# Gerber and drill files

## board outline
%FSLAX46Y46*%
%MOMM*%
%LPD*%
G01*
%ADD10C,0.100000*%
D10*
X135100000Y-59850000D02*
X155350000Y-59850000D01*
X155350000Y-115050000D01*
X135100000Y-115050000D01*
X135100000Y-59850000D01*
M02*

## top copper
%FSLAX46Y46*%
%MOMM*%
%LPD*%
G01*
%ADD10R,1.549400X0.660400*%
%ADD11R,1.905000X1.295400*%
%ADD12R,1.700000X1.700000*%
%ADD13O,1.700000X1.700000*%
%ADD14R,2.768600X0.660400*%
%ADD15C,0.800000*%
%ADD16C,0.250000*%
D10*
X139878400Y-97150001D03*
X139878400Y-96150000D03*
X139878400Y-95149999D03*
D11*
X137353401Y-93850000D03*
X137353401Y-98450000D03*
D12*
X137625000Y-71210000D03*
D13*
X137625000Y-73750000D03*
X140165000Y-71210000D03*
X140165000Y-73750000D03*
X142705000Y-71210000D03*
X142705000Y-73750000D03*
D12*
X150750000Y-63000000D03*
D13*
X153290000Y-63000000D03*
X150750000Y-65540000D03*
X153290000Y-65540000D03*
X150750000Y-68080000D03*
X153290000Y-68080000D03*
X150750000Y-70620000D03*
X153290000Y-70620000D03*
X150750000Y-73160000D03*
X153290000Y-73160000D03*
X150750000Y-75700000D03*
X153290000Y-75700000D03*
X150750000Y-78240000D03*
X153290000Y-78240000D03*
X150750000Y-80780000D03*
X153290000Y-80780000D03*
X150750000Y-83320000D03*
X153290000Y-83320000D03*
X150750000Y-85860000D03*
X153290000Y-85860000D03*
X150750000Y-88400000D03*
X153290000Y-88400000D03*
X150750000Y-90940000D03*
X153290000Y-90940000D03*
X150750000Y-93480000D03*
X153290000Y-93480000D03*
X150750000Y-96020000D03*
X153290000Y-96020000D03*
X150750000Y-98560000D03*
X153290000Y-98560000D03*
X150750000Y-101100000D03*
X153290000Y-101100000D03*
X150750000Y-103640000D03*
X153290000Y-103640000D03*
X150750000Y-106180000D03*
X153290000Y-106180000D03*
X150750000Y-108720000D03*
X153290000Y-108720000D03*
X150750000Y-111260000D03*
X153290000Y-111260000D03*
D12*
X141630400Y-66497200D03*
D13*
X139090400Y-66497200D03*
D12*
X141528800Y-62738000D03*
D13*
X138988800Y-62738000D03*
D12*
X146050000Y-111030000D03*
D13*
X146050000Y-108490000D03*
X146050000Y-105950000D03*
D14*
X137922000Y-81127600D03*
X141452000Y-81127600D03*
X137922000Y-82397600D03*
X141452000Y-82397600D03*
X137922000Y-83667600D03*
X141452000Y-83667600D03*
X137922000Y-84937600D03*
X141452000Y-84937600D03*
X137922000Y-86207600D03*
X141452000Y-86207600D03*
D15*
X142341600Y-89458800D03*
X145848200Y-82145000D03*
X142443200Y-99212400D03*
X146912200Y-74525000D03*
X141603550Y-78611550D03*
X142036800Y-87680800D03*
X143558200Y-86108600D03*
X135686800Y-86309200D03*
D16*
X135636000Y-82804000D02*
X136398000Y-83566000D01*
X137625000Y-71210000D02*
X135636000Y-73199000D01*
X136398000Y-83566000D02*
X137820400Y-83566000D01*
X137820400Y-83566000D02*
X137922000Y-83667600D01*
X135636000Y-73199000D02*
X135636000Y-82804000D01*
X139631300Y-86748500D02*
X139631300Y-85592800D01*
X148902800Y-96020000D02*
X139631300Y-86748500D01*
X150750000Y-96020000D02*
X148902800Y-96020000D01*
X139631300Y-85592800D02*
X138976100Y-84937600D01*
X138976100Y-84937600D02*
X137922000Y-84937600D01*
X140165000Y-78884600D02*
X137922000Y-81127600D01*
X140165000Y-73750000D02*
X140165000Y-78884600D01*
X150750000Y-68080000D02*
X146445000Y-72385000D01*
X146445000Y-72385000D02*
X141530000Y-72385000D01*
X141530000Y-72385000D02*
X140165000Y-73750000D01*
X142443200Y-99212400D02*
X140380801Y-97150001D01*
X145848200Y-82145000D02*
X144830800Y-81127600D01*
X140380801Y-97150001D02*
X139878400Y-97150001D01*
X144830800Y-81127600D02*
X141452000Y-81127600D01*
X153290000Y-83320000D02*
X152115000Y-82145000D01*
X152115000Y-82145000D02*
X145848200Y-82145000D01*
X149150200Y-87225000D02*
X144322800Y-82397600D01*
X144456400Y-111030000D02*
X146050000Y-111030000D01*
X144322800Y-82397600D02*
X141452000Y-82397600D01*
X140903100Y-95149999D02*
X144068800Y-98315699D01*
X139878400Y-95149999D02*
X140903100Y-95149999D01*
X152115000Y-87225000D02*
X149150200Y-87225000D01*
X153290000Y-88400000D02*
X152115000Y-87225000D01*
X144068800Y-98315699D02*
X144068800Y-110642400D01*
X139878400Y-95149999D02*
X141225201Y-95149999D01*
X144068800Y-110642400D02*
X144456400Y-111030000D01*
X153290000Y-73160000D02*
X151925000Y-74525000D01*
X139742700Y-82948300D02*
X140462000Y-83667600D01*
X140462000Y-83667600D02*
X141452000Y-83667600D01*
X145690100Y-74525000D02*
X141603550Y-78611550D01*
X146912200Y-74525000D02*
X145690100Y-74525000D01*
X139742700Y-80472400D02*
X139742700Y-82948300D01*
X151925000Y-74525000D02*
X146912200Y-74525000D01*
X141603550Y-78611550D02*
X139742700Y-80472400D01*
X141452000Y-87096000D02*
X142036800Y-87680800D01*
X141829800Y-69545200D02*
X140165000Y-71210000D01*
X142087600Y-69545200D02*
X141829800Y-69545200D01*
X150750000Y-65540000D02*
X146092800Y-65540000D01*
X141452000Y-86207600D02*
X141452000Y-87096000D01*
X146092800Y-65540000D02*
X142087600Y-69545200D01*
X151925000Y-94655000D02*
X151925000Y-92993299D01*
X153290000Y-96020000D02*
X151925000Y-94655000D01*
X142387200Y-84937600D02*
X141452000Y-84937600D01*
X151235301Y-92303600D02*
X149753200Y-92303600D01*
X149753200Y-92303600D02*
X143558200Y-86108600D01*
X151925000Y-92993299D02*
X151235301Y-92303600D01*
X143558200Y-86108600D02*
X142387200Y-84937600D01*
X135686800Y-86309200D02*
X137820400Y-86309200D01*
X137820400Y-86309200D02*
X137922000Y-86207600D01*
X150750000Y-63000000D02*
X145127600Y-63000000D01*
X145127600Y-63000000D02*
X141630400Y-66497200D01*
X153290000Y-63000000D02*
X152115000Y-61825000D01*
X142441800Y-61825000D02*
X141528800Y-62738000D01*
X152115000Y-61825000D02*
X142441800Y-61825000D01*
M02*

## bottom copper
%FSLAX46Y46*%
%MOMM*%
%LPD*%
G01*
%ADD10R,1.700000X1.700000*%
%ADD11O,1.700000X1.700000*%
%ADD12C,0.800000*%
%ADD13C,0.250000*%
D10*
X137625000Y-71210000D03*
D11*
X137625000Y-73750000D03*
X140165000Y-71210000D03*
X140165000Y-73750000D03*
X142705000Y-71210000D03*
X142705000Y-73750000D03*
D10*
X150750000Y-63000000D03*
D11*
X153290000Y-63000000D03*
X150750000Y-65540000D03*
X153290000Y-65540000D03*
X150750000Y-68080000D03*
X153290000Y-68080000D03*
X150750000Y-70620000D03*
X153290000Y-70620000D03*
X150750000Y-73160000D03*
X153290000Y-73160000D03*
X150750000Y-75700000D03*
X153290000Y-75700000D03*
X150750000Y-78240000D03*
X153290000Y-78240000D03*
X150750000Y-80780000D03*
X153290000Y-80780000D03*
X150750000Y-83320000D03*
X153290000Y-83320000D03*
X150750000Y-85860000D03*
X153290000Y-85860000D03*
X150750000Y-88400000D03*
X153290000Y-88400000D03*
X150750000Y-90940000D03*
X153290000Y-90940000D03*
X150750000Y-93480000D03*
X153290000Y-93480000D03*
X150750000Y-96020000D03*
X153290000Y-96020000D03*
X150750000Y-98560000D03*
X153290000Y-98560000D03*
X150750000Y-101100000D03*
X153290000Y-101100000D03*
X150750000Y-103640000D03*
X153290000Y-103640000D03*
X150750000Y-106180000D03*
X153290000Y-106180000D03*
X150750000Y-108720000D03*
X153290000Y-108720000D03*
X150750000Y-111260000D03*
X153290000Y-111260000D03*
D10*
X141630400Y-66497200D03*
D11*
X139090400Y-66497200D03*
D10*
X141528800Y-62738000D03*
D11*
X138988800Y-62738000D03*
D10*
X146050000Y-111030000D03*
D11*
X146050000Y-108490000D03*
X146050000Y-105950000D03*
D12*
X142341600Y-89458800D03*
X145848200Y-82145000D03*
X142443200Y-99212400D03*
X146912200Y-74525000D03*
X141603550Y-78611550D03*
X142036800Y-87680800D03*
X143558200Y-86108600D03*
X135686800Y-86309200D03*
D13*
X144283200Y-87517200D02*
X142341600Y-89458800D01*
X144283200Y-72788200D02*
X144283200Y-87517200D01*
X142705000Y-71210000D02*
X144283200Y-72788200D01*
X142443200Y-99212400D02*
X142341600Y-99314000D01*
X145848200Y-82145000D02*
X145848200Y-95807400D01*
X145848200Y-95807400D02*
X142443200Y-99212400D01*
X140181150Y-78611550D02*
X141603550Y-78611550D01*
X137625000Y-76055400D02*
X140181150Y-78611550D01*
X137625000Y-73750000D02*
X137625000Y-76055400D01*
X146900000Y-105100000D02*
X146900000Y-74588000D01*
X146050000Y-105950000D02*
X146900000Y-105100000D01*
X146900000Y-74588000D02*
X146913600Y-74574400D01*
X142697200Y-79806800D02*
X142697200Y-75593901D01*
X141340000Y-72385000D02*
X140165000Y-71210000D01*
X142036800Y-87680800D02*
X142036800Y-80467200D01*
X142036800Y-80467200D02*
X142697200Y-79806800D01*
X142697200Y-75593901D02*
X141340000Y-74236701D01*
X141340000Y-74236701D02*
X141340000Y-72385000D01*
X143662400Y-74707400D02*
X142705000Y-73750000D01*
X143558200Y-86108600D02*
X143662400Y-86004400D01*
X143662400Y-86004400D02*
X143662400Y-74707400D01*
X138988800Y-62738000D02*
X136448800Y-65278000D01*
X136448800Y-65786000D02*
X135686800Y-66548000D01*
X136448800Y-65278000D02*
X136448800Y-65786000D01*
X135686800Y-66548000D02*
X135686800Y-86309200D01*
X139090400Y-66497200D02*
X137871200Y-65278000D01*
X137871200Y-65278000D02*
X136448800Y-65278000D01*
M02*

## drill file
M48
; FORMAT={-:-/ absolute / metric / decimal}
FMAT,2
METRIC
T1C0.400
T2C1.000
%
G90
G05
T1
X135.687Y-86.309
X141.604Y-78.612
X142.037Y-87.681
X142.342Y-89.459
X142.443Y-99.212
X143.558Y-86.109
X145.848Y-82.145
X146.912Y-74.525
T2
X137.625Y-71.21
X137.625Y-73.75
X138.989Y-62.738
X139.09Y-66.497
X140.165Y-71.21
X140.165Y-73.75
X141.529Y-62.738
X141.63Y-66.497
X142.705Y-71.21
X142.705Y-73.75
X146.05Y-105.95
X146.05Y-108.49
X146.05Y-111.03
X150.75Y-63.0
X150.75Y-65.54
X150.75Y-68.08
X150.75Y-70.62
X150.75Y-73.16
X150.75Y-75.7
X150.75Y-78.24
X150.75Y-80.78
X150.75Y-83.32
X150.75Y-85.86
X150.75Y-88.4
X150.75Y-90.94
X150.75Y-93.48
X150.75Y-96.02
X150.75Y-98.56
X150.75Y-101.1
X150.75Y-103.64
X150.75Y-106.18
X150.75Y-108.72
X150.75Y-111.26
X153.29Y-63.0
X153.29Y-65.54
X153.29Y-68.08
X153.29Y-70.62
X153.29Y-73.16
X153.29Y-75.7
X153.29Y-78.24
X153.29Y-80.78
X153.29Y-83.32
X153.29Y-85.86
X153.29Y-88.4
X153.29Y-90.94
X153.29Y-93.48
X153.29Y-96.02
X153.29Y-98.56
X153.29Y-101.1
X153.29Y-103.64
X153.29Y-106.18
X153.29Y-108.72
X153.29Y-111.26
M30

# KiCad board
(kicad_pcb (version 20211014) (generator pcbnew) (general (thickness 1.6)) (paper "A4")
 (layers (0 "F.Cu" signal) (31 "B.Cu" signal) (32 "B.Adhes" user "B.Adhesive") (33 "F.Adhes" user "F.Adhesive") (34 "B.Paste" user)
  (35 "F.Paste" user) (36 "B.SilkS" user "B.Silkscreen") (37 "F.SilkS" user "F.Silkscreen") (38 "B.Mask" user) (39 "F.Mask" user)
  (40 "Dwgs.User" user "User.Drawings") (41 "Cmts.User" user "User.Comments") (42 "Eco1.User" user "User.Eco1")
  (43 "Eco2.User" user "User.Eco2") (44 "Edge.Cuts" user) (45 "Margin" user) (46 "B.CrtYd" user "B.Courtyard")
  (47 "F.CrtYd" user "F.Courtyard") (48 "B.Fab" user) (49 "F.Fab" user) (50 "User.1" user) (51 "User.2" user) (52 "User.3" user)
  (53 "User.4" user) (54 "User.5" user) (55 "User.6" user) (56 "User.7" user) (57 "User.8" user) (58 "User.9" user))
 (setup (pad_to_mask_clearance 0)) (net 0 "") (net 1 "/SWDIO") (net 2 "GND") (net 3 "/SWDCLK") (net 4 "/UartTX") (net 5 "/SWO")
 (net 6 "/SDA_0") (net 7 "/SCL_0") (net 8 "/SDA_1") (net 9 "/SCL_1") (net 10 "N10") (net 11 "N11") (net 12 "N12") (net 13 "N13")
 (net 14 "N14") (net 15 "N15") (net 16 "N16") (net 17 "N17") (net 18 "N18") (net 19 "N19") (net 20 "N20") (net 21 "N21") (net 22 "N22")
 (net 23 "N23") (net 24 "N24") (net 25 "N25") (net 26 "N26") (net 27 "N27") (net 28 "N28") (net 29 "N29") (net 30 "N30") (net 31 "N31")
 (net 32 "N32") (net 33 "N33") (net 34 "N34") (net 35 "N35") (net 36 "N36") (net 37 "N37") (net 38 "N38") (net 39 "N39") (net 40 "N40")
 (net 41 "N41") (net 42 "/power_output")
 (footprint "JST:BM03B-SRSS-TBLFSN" (layer "F.Cu") (at 138.45 96.15 -90)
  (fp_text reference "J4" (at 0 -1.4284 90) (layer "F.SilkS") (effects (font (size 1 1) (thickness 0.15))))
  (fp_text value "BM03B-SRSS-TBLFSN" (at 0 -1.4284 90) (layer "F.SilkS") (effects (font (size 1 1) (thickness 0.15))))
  (pad "1" smd rect locked (at 1.000001 -1.4284 270) (size 0.6604 1.5494) (layers "F.Cu" "F.Paste" "F.Mask") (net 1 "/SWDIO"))
  (pad "2" smd rect locked (at 0 -1.4284 270) (size 0.6604 1.5494) (layers "F.Cu" "F.Paste" "F.Mask") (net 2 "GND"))
  (pad "3" smd rect locked (at -1.000001 -1.4284 270) (size 0.6604 1.5494) (layers "F.Cu" "F.Paste" "F.Mask") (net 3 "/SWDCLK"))
  (pad "4" smd rect locked (at -2.3 1.096599) (size 1.905 1.2954) (layers "F.Cu" "F.Paste" "F.Mask"))
  (pad "5" smd rect locked (at 2.3 1.096599) (size 1.905 1.2954) (layers "F.Cu" "F.Paste" "F.Mask")))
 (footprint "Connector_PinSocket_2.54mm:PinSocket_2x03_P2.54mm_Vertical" (layer "F.Cu") (at 137.625 71.21 90)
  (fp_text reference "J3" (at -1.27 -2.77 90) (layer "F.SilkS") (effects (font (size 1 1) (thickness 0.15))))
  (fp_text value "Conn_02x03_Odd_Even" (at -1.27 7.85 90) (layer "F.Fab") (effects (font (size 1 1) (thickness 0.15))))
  (pad "1" thru_hole rect (at 0 0 90) (size 1.7 1.7) (drill 1) (layers *.Cu *.Mask) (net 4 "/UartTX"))
  (pad "2" thru_hole oval (at -2.54 0 90) (size 1.7 1.7) (drill 1) (layers *.Cu *.Mask) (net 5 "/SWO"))
  (pad "3" thru_hole oval (at 0 2.54 90) (size 1.7 1.7) (drill 1) (layers *.Cu *.Mask) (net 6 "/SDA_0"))
  (pad "4" thru_hole oval (at -2.54 2.54 90) (size 1.7 1.7) (drill 1) (layers *.Cu *.Mask) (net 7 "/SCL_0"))
  (pad "5" thru_hole oval (at 0 5.08 90) (size 1.7 1.7) (drill 1) (layers *.Cu *.Mask) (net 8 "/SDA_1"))
  (pad "6" thru_hole oval (at -2.54 5.08 90) (size 1.7 1.7) (drill 1) (layers *.Cu *.Mask) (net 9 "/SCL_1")))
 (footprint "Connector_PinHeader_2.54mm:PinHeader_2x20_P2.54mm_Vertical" (layer "F.Cu") (at 150.75 63)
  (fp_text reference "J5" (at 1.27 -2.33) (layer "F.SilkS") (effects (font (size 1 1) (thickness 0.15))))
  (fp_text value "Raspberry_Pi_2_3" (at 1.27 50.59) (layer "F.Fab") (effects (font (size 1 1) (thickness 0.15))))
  (pad "1" thru_hole rect (at 0 0) (size 1.7 1.7) (drill 1) (layers *.Cu *.Mask) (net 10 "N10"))
  (pad "2" thru_hole oval (at 2.54 0) (size 1.7 1.7) (drill 1) (layers *.Cu *.Mask) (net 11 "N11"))
  (pad "3" thru_hole oval (at 0 2.54) (size 1.7 1.7) (drill 1) (layers *.Cu *.Mask) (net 6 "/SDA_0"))
  (pad "4" thru_hole oval (at 2.54 2.54) (size 1.7 1.7) (drill 1) (layers *.Cu *.Mask) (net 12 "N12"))
  (pad "5" thru_hole oval (at 0 5.08) (size 1.7 1.7) (drill 1) (layers *.Cu *.Mask) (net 7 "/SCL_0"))
  (pad "6" thru_hole oval (at 2.54 5.08) (size 1.7 1.7) (drill 1) (layers *.Cu *.Mask) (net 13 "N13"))
  (pad "7" thru_hole oval (at 0 7.62) (size 1.7 1.7) (drill 1) (layers *.Cu *.Mask) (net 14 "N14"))
  (pad "8" thru_hole oval (at 2.54 7.62) (size 1.7 1.7) (drill 1) (layers *.Cu *.Mask) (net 4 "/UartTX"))
  (pad "9" thru_hole oval (at 0 10.16) (size 1.7 1.7) (drill 1) (layers *.Cu *.Mask) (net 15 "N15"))
  (pad "10" thru_hole oval (at 2.54 10.16) (size 1.7 1.7) (drill 1) (layers *.Cu *.Mask) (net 5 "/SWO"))
  (pad "11" thru_hole oval (at 0 12.7) (size 1.7 1.7) (drill 1) (layers *.Cu *.Mask) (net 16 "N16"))
  (pad "12" thru_hole oval (at 2.54 12.7) (size 1.7 1.7) (drill 1) (layers *.Cu *.Mask) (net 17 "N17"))
  (pad "13" thru_hole oval (at 0 15.24) (size 1.7 1.7) (drill 1) (layers *.Cu *.Mask) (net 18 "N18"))
  (pad "14" thru_hole oval (at 2.54 15.24) (size 1.7 1.7) (drill 1) (layers *.Cu *.Mask) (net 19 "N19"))
  (pad "15" thru_hole oval (at 0 17.78) (size 1.7 1.7) (drill 1) (layers *.Cu *.Mask) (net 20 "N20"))
  (pad "16" thru_hole oval (at 2.54 17.78) (size 1.7 1.7) (drill 1) (layers *.Cu *.Mask) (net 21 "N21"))
  (pad "17" thru_hole oval (at 0 20.32) (size 1.7 1.7) (drill 1) (layers *.Cu *.Mask) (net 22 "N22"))
  (pad "18" thru_hole oval (at 2.54 20.32) (size 1.7 1.7) (drill 1) (layers *.Cu *.Mask) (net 1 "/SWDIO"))
  (pad "19" thru_hole oval (at 0 22.86) (size 1.7 1.7) (drill 1) (layers *.Cu *.Mask) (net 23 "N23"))
  (pad "20" thru_hole oval (at 2.54 22.86) (size 1.7 1.7) (drill 1) (layers *.Cu *.Mask) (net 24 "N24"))
  (pad "21" thru_hole oval (at 0 25.4) (size 1.7 1.7) (drill 1) (layers *.Cu *.Mask) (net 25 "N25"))
  (pad "22" thru_hole oval (at 2.54 25.4) (size 1.7 1.7) (drill 1) (layers *.Cu *.Mask) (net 3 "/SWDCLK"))
  (pad "23" thru_hole oval (at 0 27.94) (size 1.7 1.7) (drill 1) (layers *.Cu *.Mask) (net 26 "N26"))
  (pad "24" thru_hole oval (at 2.54 27.94) (size 1.7 1.7) (drill 1) (layers *.Cu *.Mask) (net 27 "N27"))
  (pad "25" thru_hole oval (at 0 30.48) (size 1.7 1.7) (drill 1) (layers *.Cu *.Mask) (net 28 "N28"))
  (pad "26" thru_hole oval (at 2.54 30.48) (size 1.7 1.7) (drill 1) (layers *.Cu *.Mask) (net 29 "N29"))
  (pad "27" thru_hole oval (at 0 33.02) (size 1.7 1.7) (drill 1) (layers *.Cu *.Mask) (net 8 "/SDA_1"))
  (pad "28" thru_hole oval (at 2.54 33.02) (size 1.7 1.7) (drill 1) (layers *.Cu *.Mask) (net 9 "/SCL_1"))
  (pad "29" thru_hole oval (at 0 35.56) (size 1.7 1.7) (drill 1) (layers *.Cu *.Mask) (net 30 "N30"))
  (pad "30" thru_hole oval (at 2.54 35.56) (size 1.7 1.7) (drill 1) (layers *.Cu *.Mask) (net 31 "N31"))
  (pad "31" thru_hole oval (at 0 38.1) (size 1.7 1.7) (drill 1) (layers *.Cu *.Mask) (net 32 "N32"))
  (pad "32" thru_hole oval (at 2.54 38.1) (size 1.7 1.7) (drill 1) (layers *.Cu *.Mask) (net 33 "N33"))
  (pad "33" thru_hole oval (at 0 40.64) (size 1.7 1.7) (drill 1) (layers *.Cu *.Mask) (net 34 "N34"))
  (pad "34" thru_hole oval (at 2.54 40.64) (size 1.7 1.7) (drill 1) (layers *.Cu *.Mask) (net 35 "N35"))
  (pad "35" thru_hole oval (at 0 43.18) (size 1.7 1.7) (drill 1) (layers *.Cu *.Mask) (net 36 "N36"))
  (pad "36" thru_hole oval (at 2.54 43.18) (size 1.7 1.7) (drill 1) (layers *.Cu *.Mask) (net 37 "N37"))
  (pad "37" thru_hole oval (at 0 45.72) (size 1.7 1.7) (drill 1) (layers *.Cu *.Mask) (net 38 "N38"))
  (pad "38" thru_hole oval (at 2.54 45.72) (size 1.7 1.7) (drill 1) (layers *.Cu *.Mask) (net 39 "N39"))
  (pad "39" thru_hole oval (at 0 48.26) (size 1.7 1.7) (drill 1) (layers *.Cu *.Mask) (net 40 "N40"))
  (pad "40" thru_hole oval (at 2.54 48.26) (size 1.7 1.7) (drill 1) (layers *.Cu *.Mask) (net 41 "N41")))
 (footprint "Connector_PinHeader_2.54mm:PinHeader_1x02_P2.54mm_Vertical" (layer "F.Cu") (at 141.6304 66.4972 -90)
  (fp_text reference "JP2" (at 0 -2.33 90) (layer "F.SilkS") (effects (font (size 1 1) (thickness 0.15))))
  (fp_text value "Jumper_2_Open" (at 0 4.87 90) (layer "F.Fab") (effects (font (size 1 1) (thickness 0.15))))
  (pad "1" thru_hole rect (at 0 0 270) (size 1.7 1.7) (drill 1) (layers *.Cu *.Mask) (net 10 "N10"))
  (pad "2" thru_hole oval (at 0 2.54 270) (size 1.7 1.7) (drill 1) (layers *.Cu *.Mask) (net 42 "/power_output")))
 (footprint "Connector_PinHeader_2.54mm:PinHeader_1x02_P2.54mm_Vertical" (layer "F.Cu") (at 141.5288 62.738 -90)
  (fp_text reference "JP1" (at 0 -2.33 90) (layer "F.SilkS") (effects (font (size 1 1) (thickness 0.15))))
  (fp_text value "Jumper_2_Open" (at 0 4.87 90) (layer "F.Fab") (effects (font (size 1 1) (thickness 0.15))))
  (pad "1" thru_hole rect (at 0 0 270) (size 1.7 1.7) (drill 1) (layers *.Cu *.Mask) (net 11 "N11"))
  (pad "2" thru_hole oval (at 0 2.54 270) (size 1.7 1.7) (drill 1) (layers *.Cu *.Mask) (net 42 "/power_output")))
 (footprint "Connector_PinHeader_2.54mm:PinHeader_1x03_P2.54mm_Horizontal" (layer "F.Cu") (at 146.05 111.03 180)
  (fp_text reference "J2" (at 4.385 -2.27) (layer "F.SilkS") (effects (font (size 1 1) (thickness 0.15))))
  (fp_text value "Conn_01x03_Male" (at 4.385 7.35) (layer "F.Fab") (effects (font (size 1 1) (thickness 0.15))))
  (pad "1" thru_hole rect (at 0 0 180) (size 1.7 1.7) (drill 1) (layers *.Cu *.Mask) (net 3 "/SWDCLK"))
  (pad "2" thru_hole oval (at 0 2.54 180) (size 1.7 1.7) (drill 1) (layers *.Cu *.Mask) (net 2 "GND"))
  (pad "3" thru_hole oval (at 0 5.08 180) (size 1.7 1.7) (drill 1) (layers *.Cu *.Mask) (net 5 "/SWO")))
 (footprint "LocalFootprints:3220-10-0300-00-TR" (layer "F.Cu") (at 139.687 83.6676 -90)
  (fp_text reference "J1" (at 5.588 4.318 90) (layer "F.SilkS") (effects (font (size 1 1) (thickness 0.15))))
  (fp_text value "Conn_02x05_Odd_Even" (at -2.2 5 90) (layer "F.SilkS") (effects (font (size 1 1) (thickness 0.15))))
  (pad "1" smd rect (at -2.54 1.765 270) (size 0.6604 2.7686) (layers "F.Cu" "F.Paste" "F.Mask") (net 7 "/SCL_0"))
  (pad "2" smd rect (at -2.54 -1.765 270) (size 0.6604 2.7686) (layers "F.Cu" "F.Paste" "F.Mask") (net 1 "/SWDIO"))
  (pad "3" smd rect (at -1.27 1.765 270) (size 0.6604 2.7686) (layers "F.Cu" "F.Paste" "F.Mask") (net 2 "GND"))
  (pad "4" smd rect (at -1.27 -1.765 270) (size 0.6604 2.7686) (layers "F.Cu" "F.Paste" "F.Mask") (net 3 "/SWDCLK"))
  (pad "5" smd rect (at 0 1.765 270) (size 0.6604 2.7686) (layers "F.Cu" "F.Paste" "F.Mask") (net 4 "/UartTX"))
  (pad "6" smd rect (at 0 -1.765 270) (size 0.6604 2.7686) (layers "F.Cu" "F.Paste" "F.Mask") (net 5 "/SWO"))
  (pad "7" smd rect (at 1.27 1.765 270) (size 0.6604 2.7686) (layers "F.Cu" "F.Paste" "F.Mask") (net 8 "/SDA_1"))
  (pad "8" smd rect (at 1.27 -1.765 270) (size 0.6604 2.7686) (layers "F.Cu" "F.Paste" "F.Mask") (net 9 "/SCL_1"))
  (pad "9" smd rect (at 2.54 1.765 270) (size 0.6604 2.7686) (layers "F.Cu" "F.Paste" "F.Mask") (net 42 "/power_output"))
  (pad "10" smd rect (at 2.54 -1.765 270) (size 0.6604 2.7686) (layers "F.Cu" "F.Paste" "F.Mask") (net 6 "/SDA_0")))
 (gr_rect (start 135.1 59.85) (end 155.35 115.05) (layer "Edge.Cuts") (width 0.1) (fill none))
 (segment (start 135.636 82.804) (end 136.398 83.566) (width 0.25) (layer "F.Cu") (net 4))
 (segment (start 137.625 71.21) (end 135.636 73.199) (width 0.25) (layer "F.Cu") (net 4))
 (segment (start 136.398 83.566) (end 137.8204 83.566) (width 0.25) (layer "F.Cu") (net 4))
 (segment (start 137.8204 83.566) (end 137.922 83.6676) (width 0.25) (layer "F.Cu") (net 4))
 (segment (start 135.636 73.199) (end 135.636 82.804) (width 0.25) (layer "F.Cu") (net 4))
 (segment (start 139.6313 86.7485) (end 139.6313 85.5928) (width 0.25) (layer "F.Cu") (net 8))
 (segment (start 148.9028 96.02) (end 139.6313 86.7485) (width 0.25) (layer "F.Cu") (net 8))
 (segment (start 150.75 96.02) (end 148.9028 96.02) (width 0.25) (layer "F.Cu") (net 8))
 (segment (start 139.6313 85.5928) (end 138.9761 84.9376) (width 0.25) (layer "F.Cu") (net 8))
 (segment (start 138.9761 84.9376) (end 137.922 84.9376) (width 0.25) (layer "F.Cu") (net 8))
 (via (at 142.3416 89.4588) (size 0.8) (drill 0.4) (layers "F.Cu" "B.Cu") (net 8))
 (segment (start 144.2832 87.5172) (end 142.3416 89.4588) (width 0.25) (layer "B.Cu") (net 8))
 (segment (start 144.2832 72.7882) (end 144.2832 87.5172) (width 0.25) (layer "B.Cu") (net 8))
 (segment (start 142.705 71.21) (end 144.2832 72.7882) (width 0.25) (layer "B.Cu") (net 8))
 (segment (start 140.165 78.8846) (end 137.922 81.1276) (width 0.25) (layer "F.Cu") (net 7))
 (segment (start 140.165 73.75) (end 140.165 78.8846) (width 0.25) (layer "F.Cu") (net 7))
 (segment (start 150.75 68.08) (end 146.445 72.385) (width 0.25) (layer "F.Cu") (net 7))
 (segment (start 146.445 72.385) (end 141.53 72.385) (width 0.25) (layer "F.Cu") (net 7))
 (segment (start 141.53 72.385) (end 140.165 73.75) (width 0.25) (layer "F.Cu") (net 7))
 (segment (start 142.4432 99.2124) (end 140.380801 97.150001) (width 0.25) (layer "F.Cu") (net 1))
 (segment (start 145.8482 82.145) (end 144.8308 81.1276) (width 0.25) (layer "F.Cu") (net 1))
 (segment (start 140.380801 97.150001) (end 139.8784 97.150001) (width 0.25) (layer "F.Cu") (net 1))
 (segment (start 144.8308 81.1276) (end 141.452 81.1276) (width 0.25) (layer "F.Cu") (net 1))
 (segment (start 153.29 83.32) (end 152.115 82.145) (width 0.25) (layer "F.Cu") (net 1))
 (segment (start 152.115 82.145) (end 145.8482 82.145) (width 0.25) (layer "F.Cu") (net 1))
 (via (at 145.8482 82.145) (size 0.8) (drill 0.4) (layers "F.Cu" "B.Cu") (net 1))
 (via (at 142.4432 99.2124) (size 0.8) (drill 0.4) (layers "F.Cu" "B.Cu") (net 1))
 (segment (start 142.4432 99.2124) (end 142.3416 99.314) (width 0.25) (layer "B.Cu") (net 1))
 (segment (start 145.8482 82.145) (end 145.8482 95.8074) (width 0.25) (layer "B.Cu") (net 1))
 (segment (start 145.8482 95.8074) (end 142.4432 99.2124) (width 0.25) (layer "B.Cu") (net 1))
 (segment (start 149.1502 87.225) (end 144.3228 82.3976) (width 0.25) (layer "F.Cu") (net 3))
 (segment (start 144.4564 111.03) (end 146.05 111.03) (width 0.25) (layer "F.Cu") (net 3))
 (segment (start 144.3228 82.3976) (end 141.452 82.3976) (width 0.25) (layer "F.Cu") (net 3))
 (segment (start 140.9031 95.149999) (end 144.0688 98.315699) (width 0.25) (layer "F.Cu") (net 3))
 (segment (start 139.8784 95.149999) (end 140.9031 95.149999) (width 0.25) (layer "F.Cu") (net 3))
 (segment (start 152.115 87.225) (end 149.1502 87.225) (width 0.25) (layer "F.Cu") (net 3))
 (segment (start 153.29 88.4) (end 152.115 87.225) (width 0.25) (layer "F.Cu") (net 3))
 (segment (start 144.0688 98.315699) (end 144.0688 110.6424) (width 0.25) (layer "F.Cu") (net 3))
 (segment (start 139.8784 95.149999) (end 141.225201 95.149999) (width 0.25) (layer "F.Cu") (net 3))
 (segment (start 144.0688 110.6424) (end 144.4564 111.03) (width 0.25) (layer "F.Cu") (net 3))
 (segment (start 153.29 73.16) (end 151.925 74.525) (width 0.25) (layer "F.Cu") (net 5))
 (segment (start 139.7427 82.9483) (end 140.462 83.6676) (width 0.25) (layer "F.Cu") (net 5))
 (segment (start 140.462 83.6676) (end 141.452 83.6676) (width 0.25) (layer "F.Cu") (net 5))
 (segment (start 145.6901 74.525) (end 141.60355 78.61155) (width 0.25) (layer "F.Cu") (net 5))
 (segment (start 146.9122 74.525) (end 145.6901 74.525) (width 0.25) (layer "F.Cu") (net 5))
 (segment (start 139.7427 80.4724) (end 139.7427 82.9483) (width 0.25) (layer "F.Cu") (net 5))
 (segment (start 151.925 74.525) (end 146.9122 74.525) (width 0.25) (layer "F.Cu") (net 5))
 (segment (start 141.60355 78.61155) (end 139.7427 80.4724) (width 0.25) (layer "F.Cu") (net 5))
 (via (at 146.9122 74.525) (size 0.8) (drill 0.4) (layers "F.Cu" "B.Cu") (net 5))
 (via (at 141.60355 78.61155) (size 0.8) (drill 0.4) (layers "F.Cu" "B.Cu") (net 5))
 (segment (start 140.18115 78.61155) (end 141.60355 78.61155) (width 0.25) (layer "B.Cu") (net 5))
 (segment (start 137.625 76.0554) (end 140.18115 78.61155) (width 0.25) (layer "B.Cu") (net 5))
 (segment (start 137.625 73.75) (end 137.625 76.0554) (width 0.25) (layer "B.Cu") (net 5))
 (segment (start 146.9 105.1) (end 146.9 74.588) (width 0.25) (layer "B.Cu") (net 5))
 (segment (start 146.05 105.95) (end 146.9 105.1) (width 0.25) (layer "B.Cu") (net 5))
 (segment (start 146.9 74.588) (end 146.9136 74.5744) (width 0.25) (layer "B.Cu") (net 5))
 (segment (start 141.452 87.096) (end 142.0368 87.6808) (width 0.25) (layer "F.Cu") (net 6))
 (segment (start 141.8298 69.5452) (end 140.165 71.21) (width 0.25) (layer "F.Cu") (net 6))
 (segment (start 142.0876 69.5452) (end 141.8298 69.5452) (width 0.25) (layer "F.Cu") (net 6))
 (segment (start 150.75 65.54) (end 146.0928 65.54) (width 0.25) (layer "F.Cu") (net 6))
 (segment (start 141.452 86.2076) (end 141.452 87.096) (width 0.25) (layer "F.Cu") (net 6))
 (segment (start 146.0928 65.54) (end 142.0876 69.5452) (width 0.25) (layer "F.Cu") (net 6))
 (via (at 142.0368 87.6808) (size 0.8) (drill 0.4) (layers "F.Cu" "B.Cu") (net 6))
 (segment (start 142.6972 79.8068) (end 142.6972 75.593901) (width 0.25) (layer "B.Cu") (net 6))
 (segment (start 141.34 72.385) (end 140.165 71.21) (width 0.25) (layer "B.Cu") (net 6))
 (segment (start 142.0368 87.6808) (end 142.0368 80.4672) (width 0.25) (layer "B.Cu") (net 6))
 (segment (start 142.0368 80.4672) (end 142.6972 79.8068) (width 0.25) (layer "B.Cu") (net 6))
 (segment (start 142.6972 75.593901) (end 141.34 74.236701) (width 0.25) (layer "B.Cu") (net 6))
 (segment (start 141.34 74.236701) (end 141.34 72.385) (width 0.25) (layer "B.Cu") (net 6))
 (segment (start 151.925 94.655) (end 151.925 92.993299) (width 0.25) (layer "F.Cu") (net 9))
 (segment (start 153.29 96.02) (end 151.925 94.655) (width 0.25) (layer "F.Cu") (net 9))
 (segment (start 142.3872 84.9376) (end 141.452 84.9376) (width 0.25) (layer "F.Cu") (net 9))
 (segment (start 151.235301 92.3036) (end 149.7532 92.3036) (width 0.25) (layer "F.Cu") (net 9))
 (segment (start 149.7532 92.3036) (end 143.5582 86.1086) (width 0.25) (layer "F.Cu") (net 9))
 (segment (start 151.925 92.993299) (end 151.235301 92.3036) (width 0.25) (layer "F.Cu") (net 9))
 (segment (start 143.5582 86.1086) (end 142.3872 84.9376) (width 0.25) (layer "F.Cu") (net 9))
 (via (at 143.5582 86.1086) (size 0.8) (drill 0.4) (layers "F.Cu" "B.Cu") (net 9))
 (segment (start 143.6624 74.7074) (end 142.705 73.75) (width 0.25) (layer "B.Cu") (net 9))
 (segment (start 143.5582 86.1086) (end 143.6624 86.0044) (width 0.25) (layer "B.Cu") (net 9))
 (segment (start 143.6624 86.0044) (end 143.6624 74.7074) (width 0.25) (layer "B.Cu") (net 9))
 (segment (start 135.6868 86.3092) (end 137.8204 86.3092) (width 0.25) (layer "F.Cu") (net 42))
 (segment (start 137.8204 86.3092) (end 137.922 86.2076) (width 0.25) (layer "F.Cu") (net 42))
 (via (at 135.6868 86.3092) (size 0.8) (drill 0.4) (layers "F.Cu" "B.Cu") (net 42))
 (segment (start 138.9888 62.738) (end 136.4488 65.278) (width 0.25) (layer "B.Cu") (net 42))
 (segment (start 136.4488 65.786) (end 135.6868 66.548) (width 0.25) (layer "B.Cu") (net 42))
 (segment (start 136.4488 65.278) (end 136.4488 65.786) (width 0.25) (layer "B.Cu") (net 42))
 (segment (start 135.6868 66.548) (end 135.6868 86.3092) (width 0.25) (layer "B.Cu") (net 42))
 (segment (start 139.0904 66.4972) (end 137.8712 65.278) (width 0.25) (layer "B.Cu") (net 42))
 (segment (start 137.8712 65.278) (end 136.4488 65.278) (width 0.25) (layer "B.Cu") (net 42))
 (segment (start 150.75 63) (end 145.1276 63) (width 0.25) (layer "F.Cu") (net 10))
 (segment (start 145.1276 63) (end 141.6304 66.4972) (width 0.25) (layer "F.Cu") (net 10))
 (segment (start 153.29 63) (end 152.115 61.825) (width 0.25) (layer "F.Cu") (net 11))
 (segment (start 142.4418 61.825) (end 141.5288 62.738) (width 0.25) (layer "F.Cu") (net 11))
 (segment (start 152.115 61.825) (end 142.4418 61.825) (width 0.25) (layer "F.Cu") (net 11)))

